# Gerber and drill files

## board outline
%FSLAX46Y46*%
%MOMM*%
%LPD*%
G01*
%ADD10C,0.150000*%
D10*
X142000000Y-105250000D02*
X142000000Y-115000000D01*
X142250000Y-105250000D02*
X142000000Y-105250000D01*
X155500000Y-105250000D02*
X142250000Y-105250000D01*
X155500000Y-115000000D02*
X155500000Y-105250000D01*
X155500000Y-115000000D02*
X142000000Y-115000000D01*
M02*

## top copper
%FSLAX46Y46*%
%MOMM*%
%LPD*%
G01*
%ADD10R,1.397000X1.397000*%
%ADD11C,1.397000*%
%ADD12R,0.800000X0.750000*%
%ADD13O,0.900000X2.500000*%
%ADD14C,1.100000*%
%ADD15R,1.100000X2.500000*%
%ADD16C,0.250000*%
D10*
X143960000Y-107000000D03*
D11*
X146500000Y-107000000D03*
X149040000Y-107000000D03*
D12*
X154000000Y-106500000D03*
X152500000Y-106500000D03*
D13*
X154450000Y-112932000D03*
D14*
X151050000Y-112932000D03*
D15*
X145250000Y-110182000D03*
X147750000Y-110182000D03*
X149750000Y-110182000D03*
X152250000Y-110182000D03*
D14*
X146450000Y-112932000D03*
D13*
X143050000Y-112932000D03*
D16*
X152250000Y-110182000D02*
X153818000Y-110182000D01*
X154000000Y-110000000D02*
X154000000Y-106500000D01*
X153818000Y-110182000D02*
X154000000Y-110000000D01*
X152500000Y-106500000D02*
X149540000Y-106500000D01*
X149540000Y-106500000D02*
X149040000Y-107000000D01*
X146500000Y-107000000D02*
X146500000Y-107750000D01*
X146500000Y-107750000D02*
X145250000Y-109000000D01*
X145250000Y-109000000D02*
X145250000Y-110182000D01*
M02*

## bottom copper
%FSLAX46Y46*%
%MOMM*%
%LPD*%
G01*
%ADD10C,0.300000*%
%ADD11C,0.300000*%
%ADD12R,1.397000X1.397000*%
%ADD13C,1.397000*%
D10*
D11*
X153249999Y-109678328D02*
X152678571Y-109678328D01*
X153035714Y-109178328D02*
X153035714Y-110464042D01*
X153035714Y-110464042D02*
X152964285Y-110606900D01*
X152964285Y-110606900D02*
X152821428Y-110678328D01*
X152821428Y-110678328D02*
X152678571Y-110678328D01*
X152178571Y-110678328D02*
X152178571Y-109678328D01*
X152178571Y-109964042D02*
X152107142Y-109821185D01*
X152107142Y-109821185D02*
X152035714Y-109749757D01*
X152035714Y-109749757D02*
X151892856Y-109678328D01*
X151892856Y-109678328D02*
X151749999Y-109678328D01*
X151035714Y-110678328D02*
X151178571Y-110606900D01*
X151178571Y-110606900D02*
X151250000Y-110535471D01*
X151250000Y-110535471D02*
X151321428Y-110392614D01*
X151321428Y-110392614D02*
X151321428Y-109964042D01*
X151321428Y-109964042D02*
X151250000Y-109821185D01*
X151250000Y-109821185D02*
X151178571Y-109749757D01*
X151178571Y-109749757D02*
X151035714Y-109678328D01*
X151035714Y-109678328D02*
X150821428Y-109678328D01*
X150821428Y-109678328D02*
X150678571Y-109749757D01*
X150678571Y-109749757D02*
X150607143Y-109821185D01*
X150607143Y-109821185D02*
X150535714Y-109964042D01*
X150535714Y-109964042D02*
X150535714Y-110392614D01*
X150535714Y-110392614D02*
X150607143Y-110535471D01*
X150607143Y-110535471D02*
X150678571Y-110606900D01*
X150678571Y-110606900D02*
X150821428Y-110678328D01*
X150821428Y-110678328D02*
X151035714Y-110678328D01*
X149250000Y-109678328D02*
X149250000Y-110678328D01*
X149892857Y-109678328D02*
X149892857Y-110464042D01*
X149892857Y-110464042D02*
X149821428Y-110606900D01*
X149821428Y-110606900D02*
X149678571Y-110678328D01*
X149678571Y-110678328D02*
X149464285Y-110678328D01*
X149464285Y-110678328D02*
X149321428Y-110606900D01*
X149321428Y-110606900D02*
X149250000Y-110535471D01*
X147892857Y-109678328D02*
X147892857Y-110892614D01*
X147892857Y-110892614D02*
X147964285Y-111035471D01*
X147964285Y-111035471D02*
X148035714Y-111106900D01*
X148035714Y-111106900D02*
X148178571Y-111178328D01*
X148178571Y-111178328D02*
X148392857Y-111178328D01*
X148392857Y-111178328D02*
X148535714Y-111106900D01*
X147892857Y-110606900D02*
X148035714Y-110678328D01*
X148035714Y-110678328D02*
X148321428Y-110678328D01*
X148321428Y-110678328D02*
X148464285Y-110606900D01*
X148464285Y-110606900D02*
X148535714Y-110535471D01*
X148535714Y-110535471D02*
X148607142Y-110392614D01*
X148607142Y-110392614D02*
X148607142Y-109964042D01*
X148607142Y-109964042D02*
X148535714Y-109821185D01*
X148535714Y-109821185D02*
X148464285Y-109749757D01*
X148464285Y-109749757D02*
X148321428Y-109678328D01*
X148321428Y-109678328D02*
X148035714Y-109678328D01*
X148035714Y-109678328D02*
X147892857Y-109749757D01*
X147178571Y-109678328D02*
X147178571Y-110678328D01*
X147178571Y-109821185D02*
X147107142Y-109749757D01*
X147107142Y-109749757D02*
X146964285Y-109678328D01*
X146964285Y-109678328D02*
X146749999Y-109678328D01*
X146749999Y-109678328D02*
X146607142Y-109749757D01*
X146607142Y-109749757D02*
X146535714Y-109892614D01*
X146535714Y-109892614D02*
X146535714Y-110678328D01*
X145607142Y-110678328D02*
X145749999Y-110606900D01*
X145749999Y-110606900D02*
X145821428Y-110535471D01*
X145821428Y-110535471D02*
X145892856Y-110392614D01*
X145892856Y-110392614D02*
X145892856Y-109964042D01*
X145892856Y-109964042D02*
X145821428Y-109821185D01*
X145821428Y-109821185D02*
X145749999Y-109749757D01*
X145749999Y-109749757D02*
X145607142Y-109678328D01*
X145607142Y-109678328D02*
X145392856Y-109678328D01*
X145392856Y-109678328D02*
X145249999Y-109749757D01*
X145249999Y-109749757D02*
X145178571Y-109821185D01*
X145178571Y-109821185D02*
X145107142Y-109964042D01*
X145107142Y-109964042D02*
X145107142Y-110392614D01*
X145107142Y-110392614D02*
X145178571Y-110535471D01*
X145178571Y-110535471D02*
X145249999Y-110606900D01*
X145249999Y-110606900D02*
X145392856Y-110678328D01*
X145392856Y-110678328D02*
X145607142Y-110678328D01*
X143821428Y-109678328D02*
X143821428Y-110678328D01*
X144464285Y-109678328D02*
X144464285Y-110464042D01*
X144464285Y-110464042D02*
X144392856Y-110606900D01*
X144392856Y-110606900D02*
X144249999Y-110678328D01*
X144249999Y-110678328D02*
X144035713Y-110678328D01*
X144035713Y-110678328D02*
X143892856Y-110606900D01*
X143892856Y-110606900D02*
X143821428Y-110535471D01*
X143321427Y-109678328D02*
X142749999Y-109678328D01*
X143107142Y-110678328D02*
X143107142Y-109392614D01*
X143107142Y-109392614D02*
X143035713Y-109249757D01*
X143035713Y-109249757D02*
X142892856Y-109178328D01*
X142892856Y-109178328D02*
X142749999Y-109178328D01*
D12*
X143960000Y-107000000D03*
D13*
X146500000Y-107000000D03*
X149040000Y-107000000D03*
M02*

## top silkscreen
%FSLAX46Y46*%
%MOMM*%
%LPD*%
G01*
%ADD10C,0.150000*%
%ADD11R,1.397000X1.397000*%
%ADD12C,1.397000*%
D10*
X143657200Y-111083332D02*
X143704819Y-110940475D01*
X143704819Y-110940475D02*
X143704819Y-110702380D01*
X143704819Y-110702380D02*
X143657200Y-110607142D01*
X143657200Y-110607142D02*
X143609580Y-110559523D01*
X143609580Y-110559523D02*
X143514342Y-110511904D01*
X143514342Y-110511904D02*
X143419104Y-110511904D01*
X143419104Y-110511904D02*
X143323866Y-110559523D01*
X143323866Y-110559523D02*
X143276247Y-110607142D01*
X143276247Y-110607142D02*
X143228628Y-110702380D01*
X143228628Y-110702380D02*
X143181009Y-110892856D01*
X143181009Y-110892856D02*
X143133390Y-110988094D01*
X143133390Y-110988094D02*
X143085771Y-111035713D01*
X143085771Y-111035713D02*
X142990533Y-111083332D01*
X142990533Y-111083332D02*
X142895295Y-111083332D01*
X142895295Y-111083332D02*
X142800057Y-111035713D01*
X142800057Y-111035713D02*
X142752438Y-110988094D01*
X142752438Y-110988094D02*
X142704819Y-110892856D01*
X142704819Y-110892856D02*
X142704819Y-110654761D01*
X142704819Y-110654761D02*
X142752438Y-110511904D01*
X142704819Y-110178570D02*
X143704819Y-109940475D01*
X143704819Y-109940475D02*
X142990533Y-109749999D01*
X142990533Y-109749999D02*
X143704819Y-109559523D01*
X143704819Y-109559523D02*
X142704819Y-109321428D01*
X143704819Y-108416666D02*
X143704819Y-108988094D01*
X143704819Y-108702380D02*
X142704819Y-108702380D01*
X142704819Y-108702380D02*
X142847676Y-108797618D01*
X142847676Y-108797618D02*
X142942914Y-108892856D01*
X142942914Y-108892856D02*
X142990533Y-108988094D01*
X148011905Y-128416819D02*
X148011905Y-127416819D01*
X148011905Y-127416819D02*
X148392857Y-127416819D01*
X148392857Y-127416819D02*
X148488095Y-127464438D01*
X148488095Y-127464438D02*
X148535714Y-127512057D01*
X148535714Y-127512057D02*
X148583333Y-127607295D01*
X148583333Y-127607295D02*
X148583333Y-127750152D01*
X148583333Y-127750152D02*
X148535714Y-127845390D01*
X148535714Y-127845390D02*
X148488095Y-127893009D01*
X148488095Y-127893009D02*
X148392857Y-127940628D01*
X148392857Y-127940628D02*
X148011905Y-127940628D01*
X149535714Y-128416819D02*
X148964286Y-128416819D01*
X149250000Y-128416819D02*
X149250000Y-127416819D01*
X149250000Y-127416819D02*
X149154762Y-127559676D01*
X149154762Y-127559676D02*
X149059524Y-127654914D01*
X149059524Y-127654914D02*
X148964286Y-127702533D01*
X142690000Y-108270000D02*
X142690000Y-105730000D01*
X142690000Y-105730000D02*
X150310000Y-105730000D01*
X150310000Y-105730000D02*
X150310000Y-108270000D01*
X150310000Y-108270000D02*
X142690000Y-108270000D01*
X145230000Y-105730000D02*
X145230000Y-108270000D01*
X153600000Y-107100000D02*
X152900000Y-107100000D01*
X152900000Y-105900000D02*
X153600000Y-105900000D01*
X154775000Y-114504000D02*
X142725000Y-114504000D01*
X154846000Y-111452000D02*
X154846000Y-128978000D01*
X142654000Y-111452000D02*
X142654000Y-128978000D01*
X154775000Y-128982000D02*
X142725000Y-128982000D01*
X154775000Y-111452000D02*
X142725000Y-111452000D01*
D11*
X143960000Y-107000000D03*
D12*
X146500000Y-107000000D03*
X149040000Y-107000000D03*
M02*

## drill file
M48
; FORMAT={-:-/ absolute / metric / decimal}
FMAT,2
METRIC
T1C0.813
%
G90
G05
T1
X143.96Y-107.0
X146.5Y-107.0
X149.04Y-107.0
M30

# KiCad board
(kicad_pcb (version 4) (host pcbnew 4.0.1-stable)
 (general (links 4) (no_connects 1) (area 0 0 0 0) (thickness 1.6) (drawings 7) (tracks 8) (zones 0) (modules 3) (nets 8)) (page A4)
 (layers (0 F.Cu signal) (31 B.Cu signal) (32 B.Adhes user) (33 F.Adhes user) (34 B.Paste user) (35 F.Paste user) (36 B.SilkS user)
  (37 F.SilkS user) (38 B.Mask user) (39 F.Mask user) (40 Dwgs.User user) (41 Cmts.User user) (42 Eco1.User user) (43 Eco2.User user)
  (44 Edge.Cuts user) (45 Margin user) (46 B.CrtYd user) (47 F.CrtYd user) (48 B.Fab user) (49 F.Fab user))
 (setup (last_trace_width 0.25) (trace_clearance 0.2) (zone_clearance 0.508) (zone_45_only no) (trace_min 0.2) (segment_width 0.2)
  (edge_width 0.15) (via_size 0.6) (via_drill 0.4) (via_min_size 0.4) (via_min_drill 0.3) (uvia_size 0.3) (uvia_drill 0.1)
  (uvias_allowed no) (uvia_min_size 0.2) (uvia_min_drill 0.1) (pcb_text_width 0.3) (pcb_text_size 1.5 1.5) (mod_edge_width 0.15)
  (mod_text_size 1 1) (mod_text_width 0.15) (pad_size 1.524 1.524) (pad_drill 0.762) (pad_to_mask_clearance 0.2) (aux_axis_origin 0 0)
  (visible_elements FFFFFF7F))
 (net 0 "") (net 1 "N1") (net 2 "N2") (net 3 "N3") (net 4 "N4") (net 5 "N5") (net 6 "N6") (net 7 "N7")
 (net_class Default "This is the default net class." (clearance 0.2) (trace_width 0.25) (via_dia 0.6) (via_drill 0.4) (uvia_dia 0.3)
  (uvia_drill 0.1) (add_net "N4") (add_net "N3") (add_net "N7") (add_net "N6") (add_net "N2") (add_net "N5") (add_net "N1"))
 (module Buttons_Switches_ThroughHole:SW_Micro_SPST (layer F.Cu) (at 146.5 107)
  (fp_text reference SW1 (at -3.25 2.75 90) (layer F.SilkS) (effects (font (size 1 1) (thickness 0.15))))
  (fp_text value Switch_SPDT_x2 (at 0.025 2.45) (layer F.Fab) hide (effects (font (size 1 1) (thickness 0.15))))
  (fp_line (start -3.81 1.27) (end -3.81 -1.27) (layer F.SilkS) (width 0.15))
  (fp_line (start -3.81 -1.27) (end 3.81 -1.27) (layer F.SilkS) (width 0.15))
  (fp_line (start 3.81 -1.27) (end 3.81 1.27) (layer F.SilkS) (width 0.15))
  (fp_line (start 3.81 1.27) (end -3.81 1.27) (layer F.SilkS) (width 0.15))
  (fp_line (start -1.27 -1.27) (end -1.27 1.27) (layer F.SilkS) (width 0.15))
  (pad 1 thru_hole rect (at -2.54 0) (size 1.397 1.397) (drill 0.8128) (layers *.Cu *.Mask F.SilkS) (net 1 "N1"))
  (pad 2 thru_hole circle (at 0 0) (size 1.397 1.397) (drill 0.8128) (layers *.Cu *.Mask F.SilkS) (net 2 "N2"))
  (pad 3 thru_hole circle (at 2.54 0) (size 1.397 1.397) (drill 0.8128) (layers *.Cu *.Mask F.SilkS) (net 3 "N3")))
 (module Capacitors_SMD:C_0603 (layer F.Cu) (at 153.25 106.5 180)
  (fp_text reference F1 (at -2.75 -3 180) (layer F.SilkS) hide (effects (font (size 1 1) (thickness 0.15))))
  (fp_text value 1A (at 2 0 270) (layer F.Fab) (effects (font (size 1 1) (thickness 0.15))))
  (fp_line (start -0.35 -0.6) (end 0.35 -0.6) (layer F.SilkS) (width 0.15))
  (fp_line (start 0.35 0.6) (end -0.35 0.6) (layer F.SilkS) (width 0.15))
  (pad 1 smd rect (at -0.75 0 180) (size 0.8 0.75) (layers F.Cu F.Paste F.Mask) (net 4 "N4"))
  (pad 2 smd rect (at 0.75 0 180) (size 0.8 0.75) (layers F.Cu F.Paste F.Mask) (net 3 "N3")))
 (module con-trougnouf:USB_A (layer F.Cu) (at 148.75 114.5)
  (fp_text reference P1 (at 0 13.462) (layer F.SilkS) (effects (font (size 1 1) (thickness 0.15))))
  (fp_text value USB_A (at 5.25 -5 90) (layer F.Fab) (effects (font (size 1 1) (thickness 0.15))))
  (fp_line (start 6.025 0.004) (end -6.025 0.004) (layer F.SilkS) (width 0.15))
  (fp_line (start 6.096 -3.048) (end 6.096 14.478) (layer F.SilkS) (width 0.15))
  (fp_line (start -6.096 -3.048) (end -6.096 14.478) (layer F.SilkS) (width 0.15))
  (fp_line (start 6.025 14.482) (end -6.025 14.482) (layer F.SilkS) (width 0.15))
  (fp_line (start 6.025 -3.048) (end -6.025 -3.048) (layer F.SilkS) (width 0.15))
  (pad 5 smd oval (at 5.7 -1.568) (size 0.9 2.5) (layers F.Cu F.Paste F.Mask) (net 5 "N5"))
  (pad "" smd circle (at 2.3 -1.568) (size 1.1 1.1) (layers F.Cu F.Paste F.Mask))
  (pad 4 smd rect (at -3.5 -4.318) (size 1.1 2.5) (layers F.Cu F.Paste F.Mask) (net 2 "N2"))
  (pad 3 smd rect (at -1 -4.318) (size 1.1 2.5) (layers F.Cu F.Paste F.Mask) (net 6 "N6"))
  (pad 2 smd rect (at 1 -4.318) (size 1.1 2.5) (layers F.Cu F.Paste F.Mask) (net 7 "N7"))
  (pad 1 smd rect (at 3.5 -4.318) (size 1.1 2.5) (layers F.Cu F.Paste F.Mask) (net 4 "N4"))
  (pad "" smd circle (at -2.3 -1.568) (size 1.1 1.1) (layers F.Cu F.Paste F.Mask))
  (pad 5 smd oval (at -5.7 -1.568) (size 0.9 2.5) (layers F.Cu F.Paste F.Mask) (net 5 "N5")))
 (gr_line (start 142 105.25) (end 142 115) (angle 90) (layer Edge.Cuts) (width 0.15))
 (gr_line (start 142.25 105.25) (end 142 105.25) (angle 90) (layer Edge.Cuts) (width 0.15))
 (gr_line (start 155.5 105.25) (end 142.25 105.25) (angle 90) (layer Edge.Cuts) (width 0.15))
 (gr_line (start 155.5 115) (end 155.5 105.25) (angle 90) (layer Edge.Cuts) (width 0.15))
 (gr_line (start 155.5 115) (end 142 115) (angle 90) (layer Edge.Cuts) (width 0.15))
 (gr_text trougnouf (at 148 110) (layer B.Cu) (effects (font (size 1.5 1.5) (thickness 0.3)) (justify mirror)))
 (segment (start 152.25 110.182) (end 153.818 110.182) (width 0.25) (layer F.Cu) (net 4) (status 400000))
 (segment (start 154 110) (end 154 106.5) (width 0.25) (layer F.Cu) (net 4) (status 800000))
 (segment (start 153.818 110.182) (end 154 110) (width 0.25) (layer F.Cu) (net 4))
 (segment (start 152.5 106.5) (end 149.54 106.5) (width 0.25) (layer F.Cu) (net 3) (status 400000))
 (segment (start 149.54 106.5) (end 149.04 107) (width 0.25) (layer F.Cu) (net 3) (status 800000))
 (segment (start 146.5 107) (end 146.5 107.75) (width 0.25) (layer F.Cu) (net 2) (status 400000))
 (segment (start 146.5 107.75) (end 145.25 109) (width 0.25) (layer F.Cu) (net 2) (status 800000))
 (segment (start 145.25 109) (end 145.25 110.182) (width 0.25) (layer F.Cu) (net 2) (status C00000)))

